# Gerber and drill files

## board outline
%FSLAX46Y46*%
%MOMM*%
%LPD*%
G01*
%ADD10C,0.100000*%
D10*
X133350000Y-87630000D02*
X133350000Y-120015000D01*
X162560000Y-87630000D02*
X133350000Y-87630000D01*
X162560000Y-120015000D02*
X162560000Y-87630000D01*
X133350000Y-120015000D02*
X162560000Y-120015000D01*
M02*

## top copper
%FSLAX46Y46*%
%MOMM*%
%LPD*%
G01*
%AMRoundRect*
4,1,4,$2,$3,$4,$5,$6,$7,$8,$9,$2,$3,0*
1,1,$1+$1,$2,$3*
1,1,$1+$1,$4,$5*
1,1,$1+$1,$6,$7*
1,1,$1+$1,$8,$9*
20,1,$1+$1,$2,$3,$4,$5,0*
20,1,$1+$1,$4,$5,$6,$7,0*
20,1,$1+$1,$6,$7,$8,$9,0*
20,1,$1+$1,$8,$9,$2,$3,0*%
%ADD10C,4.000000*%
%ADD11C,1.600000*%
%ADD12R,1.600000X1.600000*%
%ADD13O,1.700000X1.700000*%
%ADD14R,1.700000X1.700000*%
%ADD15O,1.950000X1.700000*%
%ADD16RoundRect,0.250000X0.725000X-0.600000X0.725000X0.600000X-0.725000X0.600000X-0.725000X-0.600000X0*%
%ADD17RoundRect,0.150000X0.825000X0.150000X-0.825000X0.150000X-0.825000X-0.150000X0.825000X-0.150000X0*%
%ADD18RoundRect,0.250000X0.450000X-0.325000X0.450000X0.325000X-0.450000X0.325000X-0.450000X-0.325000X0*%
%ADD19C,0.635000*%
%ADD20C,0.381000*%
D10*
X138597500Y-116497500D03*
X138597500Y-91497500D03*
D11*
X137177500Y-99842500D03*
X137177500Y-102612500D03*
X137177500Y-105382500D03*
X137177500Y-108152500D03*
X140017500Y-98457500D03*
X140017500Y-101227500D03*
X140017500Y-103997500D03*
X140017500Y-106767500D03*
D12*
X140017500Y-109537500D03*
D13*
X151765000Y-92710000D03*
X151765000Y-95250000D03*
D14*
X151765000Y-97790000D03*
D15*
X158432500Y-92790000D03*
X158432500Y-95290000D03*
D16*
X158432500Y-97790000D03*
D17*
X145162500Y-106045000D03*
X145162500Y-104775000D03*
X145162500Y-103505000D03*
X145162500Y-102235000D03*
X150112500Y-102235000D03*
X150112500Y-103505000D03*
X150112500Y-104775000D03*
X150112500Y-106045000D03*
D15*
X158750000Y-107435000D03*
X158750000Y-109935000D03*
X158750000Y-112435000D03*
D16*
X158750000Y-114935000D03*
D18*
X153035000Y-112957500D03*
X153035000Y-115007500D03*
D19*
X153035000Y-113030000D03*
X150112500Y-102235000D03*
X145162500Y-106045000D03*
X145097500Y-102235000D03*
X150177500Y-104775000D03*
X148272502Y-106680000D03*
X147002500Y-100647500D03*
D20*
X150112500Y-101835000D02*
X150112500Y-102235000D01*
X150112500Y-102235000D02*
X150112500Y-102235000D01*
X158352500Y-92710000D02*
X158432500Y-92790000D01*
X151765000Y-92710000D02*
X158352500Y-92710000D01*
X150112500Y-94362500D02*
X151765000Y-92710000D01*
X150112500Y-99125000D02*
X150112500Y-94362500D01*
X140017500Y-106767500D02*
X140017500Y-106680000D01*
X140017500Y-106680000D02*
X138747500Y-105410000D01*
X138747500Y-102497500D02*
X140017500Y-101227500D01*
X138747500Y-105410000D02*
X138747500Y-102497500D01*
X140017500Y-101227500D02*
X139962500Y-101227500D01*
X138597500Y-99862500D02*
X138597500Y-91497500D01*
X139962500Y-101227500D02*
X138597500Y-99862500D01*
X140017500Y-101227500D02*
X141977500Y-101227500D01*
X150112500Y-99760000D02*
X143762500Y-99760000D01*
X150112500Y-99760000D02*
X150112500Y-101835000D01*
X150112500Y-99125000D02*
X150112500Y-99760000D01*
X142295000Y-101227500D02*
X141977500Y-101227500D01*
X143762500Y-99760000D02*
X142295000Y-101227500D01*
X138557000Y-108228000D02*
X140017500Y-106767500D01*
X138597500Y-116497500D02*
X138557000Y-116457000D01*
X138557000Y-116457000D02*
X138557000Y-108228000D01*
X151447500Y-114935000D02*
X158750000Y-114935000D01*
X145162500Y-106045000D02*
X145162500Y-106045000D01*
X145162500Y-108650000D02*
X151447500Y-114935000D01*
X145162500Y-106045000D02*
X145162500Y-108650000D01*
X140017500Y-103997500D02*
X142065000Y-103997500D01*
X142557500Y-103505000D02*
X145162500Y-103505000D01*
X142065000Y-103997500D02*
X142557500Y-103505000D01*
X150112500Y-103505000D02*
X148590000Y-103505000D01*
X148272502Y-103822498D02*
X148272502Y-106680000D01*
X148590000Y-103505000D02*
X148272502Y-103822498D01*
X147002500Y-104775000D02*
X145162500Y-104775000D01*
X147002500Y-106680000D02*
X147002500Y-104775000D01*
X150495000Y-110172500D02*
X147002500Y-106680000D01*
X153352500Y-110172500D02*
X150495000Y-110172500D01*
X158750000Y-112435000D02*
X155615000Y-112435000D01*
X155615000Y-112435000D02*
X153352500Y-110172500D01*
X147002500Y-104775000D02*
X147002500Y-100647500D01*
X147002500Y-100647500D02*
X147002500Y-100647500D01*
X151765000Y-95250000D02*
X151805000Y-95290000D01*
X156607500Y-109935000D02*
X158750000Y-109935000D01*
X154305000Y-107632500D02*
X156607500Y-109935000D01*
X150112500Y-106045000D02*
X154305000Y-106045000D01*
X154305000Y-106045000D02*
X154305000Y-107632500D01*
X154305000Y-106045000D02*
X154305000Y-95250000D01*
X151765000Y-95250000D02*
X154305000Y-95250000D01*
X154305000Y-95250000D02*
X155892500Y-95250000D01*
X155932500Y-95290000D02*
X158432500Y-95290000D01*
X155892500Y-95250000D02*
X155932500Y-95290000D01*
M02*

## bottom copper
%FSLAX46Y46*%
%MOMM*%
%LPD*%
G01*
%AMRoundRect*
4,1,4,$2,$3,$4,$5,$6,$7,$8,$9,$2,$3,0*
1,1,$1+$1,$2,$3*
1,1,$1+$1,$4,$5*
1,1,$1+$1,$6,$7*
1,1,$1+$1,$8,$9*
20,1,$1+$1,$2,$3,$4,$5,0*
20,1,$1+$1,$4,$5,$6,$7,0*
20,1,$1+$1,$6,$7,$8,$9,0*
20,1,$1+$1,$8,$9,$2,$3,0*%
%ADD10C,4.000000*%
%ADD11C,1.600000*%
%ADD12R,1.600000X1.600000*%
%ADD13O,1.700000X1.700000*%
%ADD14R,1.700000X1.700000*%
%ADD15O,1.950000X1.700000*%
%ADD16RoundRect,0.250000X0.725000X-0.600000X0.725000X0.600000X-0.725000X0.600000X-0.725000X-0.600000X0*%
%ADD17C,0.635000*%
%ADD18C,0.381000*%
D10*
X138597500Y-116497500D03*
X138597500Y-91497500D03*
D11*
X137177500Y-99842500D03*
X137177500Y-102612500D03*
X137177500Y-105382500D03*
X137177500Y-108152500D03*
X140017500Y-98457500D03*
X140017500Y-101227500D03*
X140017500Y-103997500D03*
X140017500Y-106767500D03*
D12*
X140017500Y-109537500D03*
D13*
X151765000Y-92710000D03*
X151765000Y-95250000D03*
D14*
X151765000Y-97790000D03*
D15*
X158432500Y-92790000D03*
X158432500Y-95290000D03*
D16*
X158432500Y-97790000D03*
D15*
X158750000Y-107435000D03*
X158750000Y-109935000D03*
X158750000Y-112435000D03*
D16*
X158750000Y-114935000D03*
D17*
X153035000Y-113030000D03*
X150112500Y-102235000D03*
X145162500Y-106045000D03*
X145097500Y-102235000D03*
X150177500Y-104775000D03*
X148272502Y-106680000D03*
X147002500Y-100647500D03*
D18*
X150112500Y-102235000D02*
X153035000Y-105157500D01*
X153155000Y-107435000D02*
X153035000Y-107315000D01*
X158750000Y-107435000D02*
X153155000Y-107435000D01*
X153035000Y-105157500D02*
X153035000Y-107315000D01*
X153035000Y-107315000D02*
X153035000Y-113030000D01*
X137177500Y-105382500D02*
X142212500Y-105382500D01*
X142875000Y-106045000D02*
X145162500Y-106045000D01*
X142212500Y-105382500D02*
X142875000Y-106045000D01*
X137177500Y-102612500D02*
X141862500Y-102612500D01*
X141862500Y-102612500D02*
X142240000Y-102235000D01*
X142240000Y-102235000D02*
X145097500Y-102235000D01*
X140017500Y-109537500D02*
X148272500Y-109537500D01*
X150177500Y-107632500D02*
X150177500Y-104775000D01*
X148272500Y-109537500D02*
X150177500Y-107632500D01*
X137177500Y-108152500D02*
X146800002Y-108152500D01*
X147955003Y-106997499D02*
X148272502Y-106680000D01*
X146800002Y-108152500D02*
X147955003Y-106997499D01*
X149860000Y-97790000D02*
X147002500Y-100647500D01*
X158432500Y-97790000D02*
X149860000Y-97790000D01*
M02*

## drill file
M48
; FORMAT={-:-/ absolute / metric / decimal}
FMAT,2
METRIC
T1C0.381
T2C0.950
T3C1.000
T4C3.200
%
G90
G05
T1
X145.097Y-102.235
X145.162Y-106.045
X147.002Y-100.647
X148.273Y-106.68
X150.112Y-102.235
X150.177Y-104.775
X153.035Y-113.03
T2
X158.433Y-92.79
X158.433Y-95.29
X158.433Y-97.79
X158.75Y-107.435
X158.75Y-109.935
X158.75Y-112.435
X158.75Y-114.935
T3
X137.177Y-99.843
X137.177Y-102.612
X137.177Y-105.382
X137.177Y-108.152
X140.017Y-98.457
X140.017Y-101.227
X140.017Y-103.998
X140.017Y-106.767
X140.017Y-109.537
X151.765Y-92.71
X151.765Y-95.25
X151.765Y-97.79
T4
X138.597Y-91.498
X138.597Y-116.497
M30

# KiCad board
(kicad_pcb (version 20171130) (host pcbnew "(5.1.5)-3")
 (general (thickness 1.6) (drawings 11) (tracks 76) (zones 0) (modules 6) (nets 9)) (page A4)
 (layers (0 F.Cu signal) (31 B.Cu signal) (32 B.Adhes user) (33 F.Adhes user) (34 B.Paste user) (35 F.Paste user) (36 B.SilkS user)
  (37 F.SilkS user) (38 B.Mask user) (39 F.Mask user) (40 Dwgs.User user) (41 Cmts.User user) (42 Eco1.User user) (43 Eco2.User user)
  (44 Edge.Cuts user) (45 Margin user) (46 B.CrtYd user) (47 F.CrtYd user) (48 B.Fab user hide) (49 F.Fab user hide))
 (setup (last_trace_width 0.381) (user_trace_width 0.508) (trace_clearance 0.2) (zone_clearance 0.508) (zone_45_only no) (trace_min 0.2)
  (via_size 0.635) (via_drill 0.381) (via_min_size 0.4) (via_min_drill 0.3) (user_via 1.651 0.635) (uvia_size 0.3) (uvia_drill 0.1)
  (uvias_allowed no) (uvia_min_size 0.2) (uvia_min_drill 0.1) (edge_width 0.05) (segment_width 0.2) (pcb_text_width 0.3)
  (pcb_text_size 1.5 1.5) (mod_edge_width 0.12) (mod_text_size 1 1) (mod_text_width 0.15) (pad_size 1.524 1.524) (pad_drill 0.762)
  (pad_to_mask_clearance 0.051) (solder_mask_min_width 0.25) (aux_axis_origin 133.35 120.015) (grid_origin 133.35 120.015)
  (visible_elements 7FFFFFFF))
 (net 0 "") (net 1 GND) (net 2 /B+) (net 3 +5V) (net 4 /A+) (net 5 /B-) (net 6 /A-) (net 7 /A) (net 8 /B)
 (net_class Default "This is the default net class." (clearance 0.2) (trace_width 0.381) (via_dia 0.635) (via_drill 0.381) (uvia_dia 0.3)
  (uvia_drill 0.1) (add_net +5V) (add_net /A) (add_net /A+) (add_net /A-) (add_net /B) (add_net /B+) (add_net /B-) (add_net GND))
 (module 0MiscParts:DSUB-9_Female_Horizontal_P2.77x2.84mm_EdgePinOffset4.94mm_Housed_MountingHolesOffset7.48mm (layer F.Cu)
  (at 140.0175 109.5375 270)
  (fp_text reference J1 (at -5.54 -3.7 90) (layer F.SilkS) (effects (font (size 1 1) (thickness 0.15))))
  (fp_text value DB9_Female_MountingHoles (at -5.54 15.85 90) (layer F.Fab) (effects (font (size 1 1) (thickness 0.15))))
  (pad 0 thru_hole circle (at 6.96 1.42 270) (size 4 4) (drill 3.2) (layers *.Cu *.Mask) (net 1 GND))
  (pad 0 thru_hole circle (at -18.04 1.42 270) (size 4 4) (drill 3.2) (layers *.Cu *.Mask) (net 1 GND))
  (pad 9 thru_hole circle (at -9.695 2.84 270) (size 1.6 1.6) (drill 1) (layers *.Cu *.Mask))
  (pad 8 thru_hole circle (at -6.925 2.84 270) (size 1.6 1.6) (drill 1) (layers *.Cu *.Mask) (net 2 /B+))
  (pad 7 thru_hole circle (at -4.155 2.84 270) (size 1.6 1.6) (drill 1) (layers *.Cu *.Mask) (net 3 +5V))
  (pad 6 thru_hole circle (at -1.385 2.84 270) (size 1.6 1.6) (drill 1) (layers *.Cu *.Mask) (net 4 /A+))
  (pad 5 thru_hole circle (at -11.08 0 270) (size 1.6 1.6) (drill 1) (layers *.Cu *.Mask))
  (pad 4 thru_hole circle (at -8.31 0 270) (size 1.6 1.6) (drill 1) (layers *.Cu *.Mask) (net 1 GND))
  (pad 3 thru_hole circle (at -5.54 0 270) (size 1.6 1.6) (drill 1) (layers *.Cu *.Mask) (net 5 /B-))
  (pad 2 thru_hole circle (at -2.77 0 270) (size 1.6 1.6) (drill 1) (layers *.Cu *.Mask) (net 1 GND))
  (pad 1 thru_hole rect (at 0 0 270) (size 1.6 1.6) (drill 1) (layers *.Cu *.Mask) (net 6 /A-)))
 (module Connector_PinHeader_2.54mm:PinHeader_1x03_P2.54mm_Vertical (layer F.Cu) (at 151.765 97.79 180)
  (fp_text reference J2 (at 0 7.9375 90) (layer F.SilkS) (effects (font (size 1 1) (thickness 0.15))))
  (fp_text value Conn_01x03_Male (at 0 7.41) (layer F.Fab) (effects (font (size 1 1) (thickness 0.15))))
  (pad 3 thru_hole oval (at 0 5.08 180) (size 1.7 1.7) (drill 1) (layers *.Cu *.Mask) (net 1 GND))
  (pad 2 thru_hole oval (at 0 2.54 180) (size 1.7 1.7) (drill 1) (layers *.Cu *.Mask) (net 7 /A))
  (pad 1 thru_hole rect (at 0 0 180) (size 1.7 1.7) (drill 1) (layers *.Cu *.Mask) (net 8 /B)))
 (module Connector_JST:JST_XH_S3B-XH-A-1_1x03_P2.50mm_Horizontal (layer F.Cu) (at 158.4325 97.79 90)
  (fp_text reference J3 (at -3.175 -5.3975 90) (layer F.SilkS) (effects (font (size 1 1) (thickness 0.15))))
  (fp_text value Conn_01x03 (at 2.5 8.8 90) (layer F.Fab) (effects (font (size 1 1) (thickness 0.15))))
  (pad 3 thru_hole oval (at 5 0 90) (size 1.7 1.95) (drill 0.95) (layers *.Cu *.Mask) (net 1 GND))
  (pad 2 thru_hole oval (at 2.5 0 90) (size 1.7 1.95) (drill 0.95) (layers *.Cu *.Mask) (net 7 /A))
  (pad 1 thru_hole roundrect (at 0 0 90) (size 1.7 1.95) (drill 0.95) (layers *.Cu *.Mask) (roundrect_rratio 0.147059) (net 8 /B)))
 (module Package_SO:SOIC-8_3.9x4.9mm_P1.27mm (layer F.Cu) (at 147.6375 104.14 180)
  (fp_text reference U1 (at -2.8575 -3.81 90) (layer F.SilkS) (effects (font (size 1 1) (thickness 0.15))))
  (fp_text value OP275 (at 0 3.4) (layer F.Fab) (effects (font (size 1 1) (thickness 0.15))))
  (pad 8 smd roundrect (at 2.475 -1.905 180) (size 1.95 0.6) (layers F.Cu F.Paste F.Mask) (roundrect_rratio 0.25) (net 3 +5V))
  (pad 7 smd roundrect (at 2.475 -0.635 180) (size 1.95 0.6) (layers F.Cu F.Paste F.Mask) (roundrect_rratio 0.25) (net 8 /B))
  (pad 6 smd roundrect (at 2.475 0.635 180) (size 1.95 0.6) (layers F.Cu F.Paste F.Mask) (roundrect_rratio 0.25) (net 5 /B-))
  (pad 5 smd roundrect (at 2.475 1.905 180) (size 1.95 0.6) (layers F.Cu F.Paste F.Mask) (roundrect_rratio 0.25) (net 2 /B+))
  (pad 4 smd roundrect (at -2.475 1.905 180) (size 1.95 0.6) (layers F.Cu F.Paste F.Mask) (roundrect_rratio 0.25) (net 1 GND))
  (pad 3 smd roundrect (at -2.475 0.635 180) (size 1.95 0.6) (layers F.Cu F.Paste F.Mask) (roundrect_rratio 0.25) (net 4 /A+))
  (pad 2 smd roundrect (at -2.475 -0.635 180) (size 1.95 0.6) (layers F.Cu F.Paste F.Mask) (roundrect_rratio 0.25) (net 6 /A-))
  (pad 1 smd roundrect (at -2.475 -1.905 180) (size 1.95 0.6) (layers F.Cu F.Paste F.Mask) (roundrect_rratio 0.25) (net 7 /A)))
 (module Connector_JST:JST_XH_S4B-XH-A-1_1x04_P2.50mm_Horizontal (layer F.Cu) (at 158.75 114.935 90)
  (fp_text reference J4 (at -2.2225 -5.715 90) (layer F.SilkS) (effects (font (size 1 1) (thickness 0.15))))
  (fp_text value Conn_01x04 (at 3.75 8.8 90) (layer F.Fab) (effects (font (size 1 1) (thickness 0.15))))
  (pad 4 thru_hole oval (at 7.5 0 90) (size 1.7 1.95) (drill 0.95) (layers *.Cu *.Mask) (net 1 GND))
  (pad 3 thru_hole oval (at 5 0 90) (size 1.7 1.95) (drill 0.95) (layers *.Cu *.Mask) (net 7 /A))
  (pad 2 thru_hole oval (at 2.5 0 90) (size 1.7 1.95) (drill 0.95) (layers *.Cu *.Mask) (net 8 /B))
  (pad 1 thru_hole roundrect (at 0 0 90) (size 1.7 1.95) (drill 0.95) (layers *.Cu *.Mask) (roundrect_rratio 0.147059) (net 3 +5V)))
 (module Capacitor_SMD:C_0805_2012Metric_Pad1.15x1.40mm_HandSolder (layer F.Cu) (at 153.035 113.9825 90)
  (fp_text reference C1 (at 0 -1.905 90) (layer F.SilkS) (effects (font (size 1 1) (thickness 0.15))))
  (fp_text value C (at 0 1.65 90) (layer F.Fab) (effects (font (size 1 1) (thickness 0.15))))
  (pad 2 smd roundrect (at 1.025 0 90) (size 1.15 1.4) (layers F.Cu F.Paste F.Mask) (roundrect_rratio 0.217391) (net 1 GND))
  (pad 1 smd roundrect (at -1.025 0 90) (size 1.15 1.4) (layers F.Cu F.Paste F.Mask) (roundrect_rratio 0.217391) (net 3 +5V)))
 (gr_line (start 133.35 87.63) (end 133.35 120.015) (layer Edge.Cuts) (width 0.1))
 (gr_line (start 162.56 87.63) (end 133.35 87.63) (layer Edge.Cuts) (width 0.1))
 (gr_line (start 162.56 120.015) (end 162.56 87.63) (layer Edge.Cuts) (width 0.1))
 (gr_line (start 133.35 120.015) (end 162.56 120.015) (layer Edge.Cuts) (width 0.1))
 (via (at 153.035 113.03) (size 0.635) (drill 0.381) (layers F.Cu B.Cu) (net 1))
 (segment (start 150.1125 101.835) (end 150.1125 102.235) (width 0.381) (layer F.Cu) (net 1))
 (segment (start 150.1125 102.235) (end 150.1125 102.235) (width 0.381) (layer F.Cu) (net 1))
 (via (at 150.1125 102.235) (size 0.635) (drill 0.381) (layers F.Cu B.Cu) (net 1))
 (segment (start 150.1125 102.235) (end 153.035 105.1575) (width 0.381) (layer B.Cu) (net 1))
 (segment (start 153.155 107.435) (end 153.035 107.315) (width 0.381) (layer B.Cu) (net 1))
 (segment (start 158.75 107.435) (end 153.155 107.435) (width 0.381) (layer B.Cu) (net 1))
 (segment (start 153.035 105.1575) (end 153.035 107.315) (width 0.381) (layer B.Cu) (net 1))
 (segment (start 153.035 107.315) (end 153.035 113.03) (width 0.381) (layer B.Cu) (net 1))
 (segment (start 158.3525 92.71) (end 158.4325 92.79) (width 0.381) (layer F.Cu) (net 1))
 (segment (start 151.765 92.71) (end 158.3525 92.71) (width 0.381) (layer F.Cu) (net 1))
 (segment (start 150.1125 94.3625) (end 151.765 92.71) (width 0.381) (layer F.Cu) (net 1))
 (segment (start 150.1125 99.125) (end 150.1125 94.3625) (width 0.381) (layer F.Cu) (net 1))
 (segment (start 140.0175 106.7675) (end 140.0175 106.68) (width 0.381) (layer F.Cu) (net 1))
 (segment (start 140.0175 106.68) (end 138.7475 105.41) (width 0.381) (layer F.Cu) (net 1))
 (segment (start 138.7475 102.4975) (end 140.0175 101.2275) (width 0.381) (layer F.Cu) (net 1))
 (segment (start 138.7475 105.41) (end 138.7475 102.4975) (width 0.381) (layer F.Cu) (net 1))
 (segment (start 140.0175 101.2275) (end 139.9625 101.2275) (width 0.381) (layer F.Cu) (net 1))
 (segment (start 138.5975 99.8625) (end 138.5975 91.4975) (width 0.381) (layer F.Cu) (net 1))
 (segment (start 139.9625 101.2275) (end 138.5975 99.8625) (width 0.381) (layer F.Cu) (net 1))
 (segment (start 140.0175 101.2275) (end 141.9775 101.2275) (width 0.381) (layer F.Cu) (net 1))
 (segment (start 150.1125 99.76) (end 143.7625 99.76) (width 0.381) (layer F.Cu) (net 1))
 (segment (start 150.1125 99.76) (end 150.1125 101.835) (width 0.381) (layer F.Cu) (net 1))
 (segment (start 150.1125 99.125) (end 150.1125 99.76) (width 0.381) (layer F.Cu) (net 1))
 (segment (start 142.295 101.2275) (end 141.9775 101.2275) (width 0.381) (layer F.Cu) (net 1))
 (segment (start 143.7625 99.76) (end 142.295 101.2275) (width 0.381) (layer F.Cu) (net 1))
 (segment (start 138.557 108.228) (end 140.0175 106.7675) (width 0.381) (layer F.Cu) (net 1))
 (segment (start 138.5975 116.4975) (end 138.557 116.457) (width 0.381) (layer F.Cu) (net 1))
 (segment (start 138.557 116.457) (end 138.557 108.228) (width 0.381) (layer F.Cu) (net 1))
 (segment (start 151.4475 114.935) (end 158.75 114.935) (width 0.381) (layer F.Cu) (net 3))
 (segment (start 145.1625 106.045) (end 145.1625 106.045) (width 0.381) (layer F.Cu) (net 3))
 (segment (start 145.1625 108.65) (end 151.4475 114.935) (width 0.381) (layer F.Cu) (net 3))
 (segment (start 145.1625 106.045) (end 145.1625 108.65) (width 0.381) (layer F.Cu) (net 3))
 (via (at 145.1625 106.045) (size 0.635) (drill 0.381) (layers F.Cu B.Cu) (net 3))
 (segment (start 137.1775 105.3825) (end 142.2125 105.3825) (width 0.381) (layer B.Cu) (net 3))
 (segment (start 142.875 106.045) (end 145.1625 106.045) (width 0.381) (layer B.Cu) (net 3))
 (segment (start 142.2125 105.3825) (end 142.875 106.045) (width 0.381) (layer B.Cu) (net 3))
 (via (at 145.0975 102.235) (size 0.635) (drill 0.381) (layers F.Cu B.Cu) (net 2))
 (segment (start 137.1775 102.6125) (end 141.8625 102.6125) (width 0.381) (layer B.Cu) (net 2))
 (segment (start 141.8625 102.6125) (end 142.24 102.235) (width 0.381) (layer B.Cu) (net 2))
 (segment (start 142.24 102.235) (end 145.0975 102.235) (width 0.381) (layer B.Cu) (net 2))
 (segment (start 140.0175 103.9975) (end 142.065 103.9975) (width 0.381) (layer F.Cu) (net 5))
 (segment (start 142.5575 103.505) (end 145.1625 103.505) (width 0.381) (layer F.Cu) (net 5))
 (segment (start 142.065 103.9975) (end 142.5575 103.505) (width 0.381) (layer F.Cu) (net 5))
 (via (at 150.1775 104.775) (size 0.635) (drill 0.381) (layers F.Cu B.Cu) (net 6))
 (segment (start 140.0175 109.5375) (end 148.2725 109.5375) (width 0.381) (layer B.Cu) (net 6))
 (segment (start 150.1775 107.6325) (end 150.1775 104.775) (width 0.381) (layer B.Cu) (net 6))
 (segment (start 148.2725 109.5375) (end 150.1775 107.6325) (width 0.381) (layer B.Cu) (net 6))
 (via (at 148.272502 106.68) (size 0.635) (drill 0.381) (layers F.Cu B.Cu) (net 4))
 (segment (start 137.1775 108.1525) (end 146.800002 108.1525) (width 0.381) (layer B.Cu) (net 4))
 (segment (start 147.955003 106.997499) (end 148.272502 106.68) (width 0.381) (layer B.Cu) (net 4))
 (segment (start 146.800002 108.1525) (end 147.955003 106.997499) (width 0.381) (layer B.Cu) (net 4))
 (segment (start 150.1125 103.505) (end 148.59 103.505) (width 0.381) (layer F.Cu) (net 4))
 (segment (start 148.272502 103.822498) (end 148.272502 106.68) (width 0.381) (layer F.Cu) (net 4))
 (segment (start 148.59 103.505) (end 148.272502 103.822498) (width 0.381) (layer F.Cu) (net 4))
 (segment (start 147.0025 104.775) (end 145.1625 104.775) (width 0.381) (layer F.Cu) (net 8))
 (segment (start 147.0025 106.68) (end 147.0025 104.775) (width 0.381) (layer F.Cu) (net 8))
 (segment (start 150.495 110.1725) (end 147.0025 106.68) (width 0.381) (layer F.Cu) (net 8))
 (segment (start 153.3525 110.1725) (end 150.495 110.1725) (width 0.381) (layer F.Cu) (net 8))
 (segment (start 158.75 112.435) (end 155.615 112.435) (width 0.381) (layer F.Cu) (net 8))
 (segment (start 155.615 112.435) (end 153.3525 110.1725) (width 0.381) (layer F.Cu) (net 8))
 (segment (start 147.0025 104.775) (end 147.0025 100.6475) (width 0.381) (layer F.Cu) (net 8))
 (segment (start 147.0025 100.6475) (end 147.0025 100.6475) (width 0.381) (layer F.Cu) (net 8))
 (via (at 147.0025 100.6475) (size 0.635) (drill 0.381) (layers F.Cu B.Cu) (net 8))
 (segment (start 149.86 97.79) (end 147.0025 100.6475) (width 0.381) (layer B.Cu) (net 8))
 (segment (start 158.4325 97.79) (end 149.86 97.79) (width 0.381) (layer B.Cu) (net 8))
 (segment (start 151.765 95.25) (end 151.805 95.29) (width 0.381) (layer F.Cu) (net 7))
 (segment (start 156.6075 109.935) (end 158.75 109.935) (width 0.381) (layer F.Cu) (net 7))
 (segment (start 154.305 107.6325) (end 156.6075 109.935) (width 0.381) (layer F.Cu) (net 7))
 (segment (start 150.1125 106.045) (end 154.305 106.045) (width 0.381) (layer F.Cu) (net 7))
 (segment (start 154.305 106.045) (end 154.305 107.6325) (width 0.381) (layer F.Cu) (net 7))
 (segment (start 154.305 106.045) (end 154.305 95.25) (width 0.381) (layer F.Cu) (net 7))
 (segment (start 151.765 95.25) (end 154.305 95.25) (width 0.381) (layer F.Cu) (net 7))
 (segment (start 154.305 95.25) (end 155.8925 95.25) (width 0.381) (layer F.Cu) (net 7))
 (segment (start 155.9325 95.29) (end 158.4325 95.29) (width 0.381) (layer F.Cu) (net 7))
 (segment (start 155.8925 95.25) (end 155.9325 95.29) (width 0.381) (layer F.Cu) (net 7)))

